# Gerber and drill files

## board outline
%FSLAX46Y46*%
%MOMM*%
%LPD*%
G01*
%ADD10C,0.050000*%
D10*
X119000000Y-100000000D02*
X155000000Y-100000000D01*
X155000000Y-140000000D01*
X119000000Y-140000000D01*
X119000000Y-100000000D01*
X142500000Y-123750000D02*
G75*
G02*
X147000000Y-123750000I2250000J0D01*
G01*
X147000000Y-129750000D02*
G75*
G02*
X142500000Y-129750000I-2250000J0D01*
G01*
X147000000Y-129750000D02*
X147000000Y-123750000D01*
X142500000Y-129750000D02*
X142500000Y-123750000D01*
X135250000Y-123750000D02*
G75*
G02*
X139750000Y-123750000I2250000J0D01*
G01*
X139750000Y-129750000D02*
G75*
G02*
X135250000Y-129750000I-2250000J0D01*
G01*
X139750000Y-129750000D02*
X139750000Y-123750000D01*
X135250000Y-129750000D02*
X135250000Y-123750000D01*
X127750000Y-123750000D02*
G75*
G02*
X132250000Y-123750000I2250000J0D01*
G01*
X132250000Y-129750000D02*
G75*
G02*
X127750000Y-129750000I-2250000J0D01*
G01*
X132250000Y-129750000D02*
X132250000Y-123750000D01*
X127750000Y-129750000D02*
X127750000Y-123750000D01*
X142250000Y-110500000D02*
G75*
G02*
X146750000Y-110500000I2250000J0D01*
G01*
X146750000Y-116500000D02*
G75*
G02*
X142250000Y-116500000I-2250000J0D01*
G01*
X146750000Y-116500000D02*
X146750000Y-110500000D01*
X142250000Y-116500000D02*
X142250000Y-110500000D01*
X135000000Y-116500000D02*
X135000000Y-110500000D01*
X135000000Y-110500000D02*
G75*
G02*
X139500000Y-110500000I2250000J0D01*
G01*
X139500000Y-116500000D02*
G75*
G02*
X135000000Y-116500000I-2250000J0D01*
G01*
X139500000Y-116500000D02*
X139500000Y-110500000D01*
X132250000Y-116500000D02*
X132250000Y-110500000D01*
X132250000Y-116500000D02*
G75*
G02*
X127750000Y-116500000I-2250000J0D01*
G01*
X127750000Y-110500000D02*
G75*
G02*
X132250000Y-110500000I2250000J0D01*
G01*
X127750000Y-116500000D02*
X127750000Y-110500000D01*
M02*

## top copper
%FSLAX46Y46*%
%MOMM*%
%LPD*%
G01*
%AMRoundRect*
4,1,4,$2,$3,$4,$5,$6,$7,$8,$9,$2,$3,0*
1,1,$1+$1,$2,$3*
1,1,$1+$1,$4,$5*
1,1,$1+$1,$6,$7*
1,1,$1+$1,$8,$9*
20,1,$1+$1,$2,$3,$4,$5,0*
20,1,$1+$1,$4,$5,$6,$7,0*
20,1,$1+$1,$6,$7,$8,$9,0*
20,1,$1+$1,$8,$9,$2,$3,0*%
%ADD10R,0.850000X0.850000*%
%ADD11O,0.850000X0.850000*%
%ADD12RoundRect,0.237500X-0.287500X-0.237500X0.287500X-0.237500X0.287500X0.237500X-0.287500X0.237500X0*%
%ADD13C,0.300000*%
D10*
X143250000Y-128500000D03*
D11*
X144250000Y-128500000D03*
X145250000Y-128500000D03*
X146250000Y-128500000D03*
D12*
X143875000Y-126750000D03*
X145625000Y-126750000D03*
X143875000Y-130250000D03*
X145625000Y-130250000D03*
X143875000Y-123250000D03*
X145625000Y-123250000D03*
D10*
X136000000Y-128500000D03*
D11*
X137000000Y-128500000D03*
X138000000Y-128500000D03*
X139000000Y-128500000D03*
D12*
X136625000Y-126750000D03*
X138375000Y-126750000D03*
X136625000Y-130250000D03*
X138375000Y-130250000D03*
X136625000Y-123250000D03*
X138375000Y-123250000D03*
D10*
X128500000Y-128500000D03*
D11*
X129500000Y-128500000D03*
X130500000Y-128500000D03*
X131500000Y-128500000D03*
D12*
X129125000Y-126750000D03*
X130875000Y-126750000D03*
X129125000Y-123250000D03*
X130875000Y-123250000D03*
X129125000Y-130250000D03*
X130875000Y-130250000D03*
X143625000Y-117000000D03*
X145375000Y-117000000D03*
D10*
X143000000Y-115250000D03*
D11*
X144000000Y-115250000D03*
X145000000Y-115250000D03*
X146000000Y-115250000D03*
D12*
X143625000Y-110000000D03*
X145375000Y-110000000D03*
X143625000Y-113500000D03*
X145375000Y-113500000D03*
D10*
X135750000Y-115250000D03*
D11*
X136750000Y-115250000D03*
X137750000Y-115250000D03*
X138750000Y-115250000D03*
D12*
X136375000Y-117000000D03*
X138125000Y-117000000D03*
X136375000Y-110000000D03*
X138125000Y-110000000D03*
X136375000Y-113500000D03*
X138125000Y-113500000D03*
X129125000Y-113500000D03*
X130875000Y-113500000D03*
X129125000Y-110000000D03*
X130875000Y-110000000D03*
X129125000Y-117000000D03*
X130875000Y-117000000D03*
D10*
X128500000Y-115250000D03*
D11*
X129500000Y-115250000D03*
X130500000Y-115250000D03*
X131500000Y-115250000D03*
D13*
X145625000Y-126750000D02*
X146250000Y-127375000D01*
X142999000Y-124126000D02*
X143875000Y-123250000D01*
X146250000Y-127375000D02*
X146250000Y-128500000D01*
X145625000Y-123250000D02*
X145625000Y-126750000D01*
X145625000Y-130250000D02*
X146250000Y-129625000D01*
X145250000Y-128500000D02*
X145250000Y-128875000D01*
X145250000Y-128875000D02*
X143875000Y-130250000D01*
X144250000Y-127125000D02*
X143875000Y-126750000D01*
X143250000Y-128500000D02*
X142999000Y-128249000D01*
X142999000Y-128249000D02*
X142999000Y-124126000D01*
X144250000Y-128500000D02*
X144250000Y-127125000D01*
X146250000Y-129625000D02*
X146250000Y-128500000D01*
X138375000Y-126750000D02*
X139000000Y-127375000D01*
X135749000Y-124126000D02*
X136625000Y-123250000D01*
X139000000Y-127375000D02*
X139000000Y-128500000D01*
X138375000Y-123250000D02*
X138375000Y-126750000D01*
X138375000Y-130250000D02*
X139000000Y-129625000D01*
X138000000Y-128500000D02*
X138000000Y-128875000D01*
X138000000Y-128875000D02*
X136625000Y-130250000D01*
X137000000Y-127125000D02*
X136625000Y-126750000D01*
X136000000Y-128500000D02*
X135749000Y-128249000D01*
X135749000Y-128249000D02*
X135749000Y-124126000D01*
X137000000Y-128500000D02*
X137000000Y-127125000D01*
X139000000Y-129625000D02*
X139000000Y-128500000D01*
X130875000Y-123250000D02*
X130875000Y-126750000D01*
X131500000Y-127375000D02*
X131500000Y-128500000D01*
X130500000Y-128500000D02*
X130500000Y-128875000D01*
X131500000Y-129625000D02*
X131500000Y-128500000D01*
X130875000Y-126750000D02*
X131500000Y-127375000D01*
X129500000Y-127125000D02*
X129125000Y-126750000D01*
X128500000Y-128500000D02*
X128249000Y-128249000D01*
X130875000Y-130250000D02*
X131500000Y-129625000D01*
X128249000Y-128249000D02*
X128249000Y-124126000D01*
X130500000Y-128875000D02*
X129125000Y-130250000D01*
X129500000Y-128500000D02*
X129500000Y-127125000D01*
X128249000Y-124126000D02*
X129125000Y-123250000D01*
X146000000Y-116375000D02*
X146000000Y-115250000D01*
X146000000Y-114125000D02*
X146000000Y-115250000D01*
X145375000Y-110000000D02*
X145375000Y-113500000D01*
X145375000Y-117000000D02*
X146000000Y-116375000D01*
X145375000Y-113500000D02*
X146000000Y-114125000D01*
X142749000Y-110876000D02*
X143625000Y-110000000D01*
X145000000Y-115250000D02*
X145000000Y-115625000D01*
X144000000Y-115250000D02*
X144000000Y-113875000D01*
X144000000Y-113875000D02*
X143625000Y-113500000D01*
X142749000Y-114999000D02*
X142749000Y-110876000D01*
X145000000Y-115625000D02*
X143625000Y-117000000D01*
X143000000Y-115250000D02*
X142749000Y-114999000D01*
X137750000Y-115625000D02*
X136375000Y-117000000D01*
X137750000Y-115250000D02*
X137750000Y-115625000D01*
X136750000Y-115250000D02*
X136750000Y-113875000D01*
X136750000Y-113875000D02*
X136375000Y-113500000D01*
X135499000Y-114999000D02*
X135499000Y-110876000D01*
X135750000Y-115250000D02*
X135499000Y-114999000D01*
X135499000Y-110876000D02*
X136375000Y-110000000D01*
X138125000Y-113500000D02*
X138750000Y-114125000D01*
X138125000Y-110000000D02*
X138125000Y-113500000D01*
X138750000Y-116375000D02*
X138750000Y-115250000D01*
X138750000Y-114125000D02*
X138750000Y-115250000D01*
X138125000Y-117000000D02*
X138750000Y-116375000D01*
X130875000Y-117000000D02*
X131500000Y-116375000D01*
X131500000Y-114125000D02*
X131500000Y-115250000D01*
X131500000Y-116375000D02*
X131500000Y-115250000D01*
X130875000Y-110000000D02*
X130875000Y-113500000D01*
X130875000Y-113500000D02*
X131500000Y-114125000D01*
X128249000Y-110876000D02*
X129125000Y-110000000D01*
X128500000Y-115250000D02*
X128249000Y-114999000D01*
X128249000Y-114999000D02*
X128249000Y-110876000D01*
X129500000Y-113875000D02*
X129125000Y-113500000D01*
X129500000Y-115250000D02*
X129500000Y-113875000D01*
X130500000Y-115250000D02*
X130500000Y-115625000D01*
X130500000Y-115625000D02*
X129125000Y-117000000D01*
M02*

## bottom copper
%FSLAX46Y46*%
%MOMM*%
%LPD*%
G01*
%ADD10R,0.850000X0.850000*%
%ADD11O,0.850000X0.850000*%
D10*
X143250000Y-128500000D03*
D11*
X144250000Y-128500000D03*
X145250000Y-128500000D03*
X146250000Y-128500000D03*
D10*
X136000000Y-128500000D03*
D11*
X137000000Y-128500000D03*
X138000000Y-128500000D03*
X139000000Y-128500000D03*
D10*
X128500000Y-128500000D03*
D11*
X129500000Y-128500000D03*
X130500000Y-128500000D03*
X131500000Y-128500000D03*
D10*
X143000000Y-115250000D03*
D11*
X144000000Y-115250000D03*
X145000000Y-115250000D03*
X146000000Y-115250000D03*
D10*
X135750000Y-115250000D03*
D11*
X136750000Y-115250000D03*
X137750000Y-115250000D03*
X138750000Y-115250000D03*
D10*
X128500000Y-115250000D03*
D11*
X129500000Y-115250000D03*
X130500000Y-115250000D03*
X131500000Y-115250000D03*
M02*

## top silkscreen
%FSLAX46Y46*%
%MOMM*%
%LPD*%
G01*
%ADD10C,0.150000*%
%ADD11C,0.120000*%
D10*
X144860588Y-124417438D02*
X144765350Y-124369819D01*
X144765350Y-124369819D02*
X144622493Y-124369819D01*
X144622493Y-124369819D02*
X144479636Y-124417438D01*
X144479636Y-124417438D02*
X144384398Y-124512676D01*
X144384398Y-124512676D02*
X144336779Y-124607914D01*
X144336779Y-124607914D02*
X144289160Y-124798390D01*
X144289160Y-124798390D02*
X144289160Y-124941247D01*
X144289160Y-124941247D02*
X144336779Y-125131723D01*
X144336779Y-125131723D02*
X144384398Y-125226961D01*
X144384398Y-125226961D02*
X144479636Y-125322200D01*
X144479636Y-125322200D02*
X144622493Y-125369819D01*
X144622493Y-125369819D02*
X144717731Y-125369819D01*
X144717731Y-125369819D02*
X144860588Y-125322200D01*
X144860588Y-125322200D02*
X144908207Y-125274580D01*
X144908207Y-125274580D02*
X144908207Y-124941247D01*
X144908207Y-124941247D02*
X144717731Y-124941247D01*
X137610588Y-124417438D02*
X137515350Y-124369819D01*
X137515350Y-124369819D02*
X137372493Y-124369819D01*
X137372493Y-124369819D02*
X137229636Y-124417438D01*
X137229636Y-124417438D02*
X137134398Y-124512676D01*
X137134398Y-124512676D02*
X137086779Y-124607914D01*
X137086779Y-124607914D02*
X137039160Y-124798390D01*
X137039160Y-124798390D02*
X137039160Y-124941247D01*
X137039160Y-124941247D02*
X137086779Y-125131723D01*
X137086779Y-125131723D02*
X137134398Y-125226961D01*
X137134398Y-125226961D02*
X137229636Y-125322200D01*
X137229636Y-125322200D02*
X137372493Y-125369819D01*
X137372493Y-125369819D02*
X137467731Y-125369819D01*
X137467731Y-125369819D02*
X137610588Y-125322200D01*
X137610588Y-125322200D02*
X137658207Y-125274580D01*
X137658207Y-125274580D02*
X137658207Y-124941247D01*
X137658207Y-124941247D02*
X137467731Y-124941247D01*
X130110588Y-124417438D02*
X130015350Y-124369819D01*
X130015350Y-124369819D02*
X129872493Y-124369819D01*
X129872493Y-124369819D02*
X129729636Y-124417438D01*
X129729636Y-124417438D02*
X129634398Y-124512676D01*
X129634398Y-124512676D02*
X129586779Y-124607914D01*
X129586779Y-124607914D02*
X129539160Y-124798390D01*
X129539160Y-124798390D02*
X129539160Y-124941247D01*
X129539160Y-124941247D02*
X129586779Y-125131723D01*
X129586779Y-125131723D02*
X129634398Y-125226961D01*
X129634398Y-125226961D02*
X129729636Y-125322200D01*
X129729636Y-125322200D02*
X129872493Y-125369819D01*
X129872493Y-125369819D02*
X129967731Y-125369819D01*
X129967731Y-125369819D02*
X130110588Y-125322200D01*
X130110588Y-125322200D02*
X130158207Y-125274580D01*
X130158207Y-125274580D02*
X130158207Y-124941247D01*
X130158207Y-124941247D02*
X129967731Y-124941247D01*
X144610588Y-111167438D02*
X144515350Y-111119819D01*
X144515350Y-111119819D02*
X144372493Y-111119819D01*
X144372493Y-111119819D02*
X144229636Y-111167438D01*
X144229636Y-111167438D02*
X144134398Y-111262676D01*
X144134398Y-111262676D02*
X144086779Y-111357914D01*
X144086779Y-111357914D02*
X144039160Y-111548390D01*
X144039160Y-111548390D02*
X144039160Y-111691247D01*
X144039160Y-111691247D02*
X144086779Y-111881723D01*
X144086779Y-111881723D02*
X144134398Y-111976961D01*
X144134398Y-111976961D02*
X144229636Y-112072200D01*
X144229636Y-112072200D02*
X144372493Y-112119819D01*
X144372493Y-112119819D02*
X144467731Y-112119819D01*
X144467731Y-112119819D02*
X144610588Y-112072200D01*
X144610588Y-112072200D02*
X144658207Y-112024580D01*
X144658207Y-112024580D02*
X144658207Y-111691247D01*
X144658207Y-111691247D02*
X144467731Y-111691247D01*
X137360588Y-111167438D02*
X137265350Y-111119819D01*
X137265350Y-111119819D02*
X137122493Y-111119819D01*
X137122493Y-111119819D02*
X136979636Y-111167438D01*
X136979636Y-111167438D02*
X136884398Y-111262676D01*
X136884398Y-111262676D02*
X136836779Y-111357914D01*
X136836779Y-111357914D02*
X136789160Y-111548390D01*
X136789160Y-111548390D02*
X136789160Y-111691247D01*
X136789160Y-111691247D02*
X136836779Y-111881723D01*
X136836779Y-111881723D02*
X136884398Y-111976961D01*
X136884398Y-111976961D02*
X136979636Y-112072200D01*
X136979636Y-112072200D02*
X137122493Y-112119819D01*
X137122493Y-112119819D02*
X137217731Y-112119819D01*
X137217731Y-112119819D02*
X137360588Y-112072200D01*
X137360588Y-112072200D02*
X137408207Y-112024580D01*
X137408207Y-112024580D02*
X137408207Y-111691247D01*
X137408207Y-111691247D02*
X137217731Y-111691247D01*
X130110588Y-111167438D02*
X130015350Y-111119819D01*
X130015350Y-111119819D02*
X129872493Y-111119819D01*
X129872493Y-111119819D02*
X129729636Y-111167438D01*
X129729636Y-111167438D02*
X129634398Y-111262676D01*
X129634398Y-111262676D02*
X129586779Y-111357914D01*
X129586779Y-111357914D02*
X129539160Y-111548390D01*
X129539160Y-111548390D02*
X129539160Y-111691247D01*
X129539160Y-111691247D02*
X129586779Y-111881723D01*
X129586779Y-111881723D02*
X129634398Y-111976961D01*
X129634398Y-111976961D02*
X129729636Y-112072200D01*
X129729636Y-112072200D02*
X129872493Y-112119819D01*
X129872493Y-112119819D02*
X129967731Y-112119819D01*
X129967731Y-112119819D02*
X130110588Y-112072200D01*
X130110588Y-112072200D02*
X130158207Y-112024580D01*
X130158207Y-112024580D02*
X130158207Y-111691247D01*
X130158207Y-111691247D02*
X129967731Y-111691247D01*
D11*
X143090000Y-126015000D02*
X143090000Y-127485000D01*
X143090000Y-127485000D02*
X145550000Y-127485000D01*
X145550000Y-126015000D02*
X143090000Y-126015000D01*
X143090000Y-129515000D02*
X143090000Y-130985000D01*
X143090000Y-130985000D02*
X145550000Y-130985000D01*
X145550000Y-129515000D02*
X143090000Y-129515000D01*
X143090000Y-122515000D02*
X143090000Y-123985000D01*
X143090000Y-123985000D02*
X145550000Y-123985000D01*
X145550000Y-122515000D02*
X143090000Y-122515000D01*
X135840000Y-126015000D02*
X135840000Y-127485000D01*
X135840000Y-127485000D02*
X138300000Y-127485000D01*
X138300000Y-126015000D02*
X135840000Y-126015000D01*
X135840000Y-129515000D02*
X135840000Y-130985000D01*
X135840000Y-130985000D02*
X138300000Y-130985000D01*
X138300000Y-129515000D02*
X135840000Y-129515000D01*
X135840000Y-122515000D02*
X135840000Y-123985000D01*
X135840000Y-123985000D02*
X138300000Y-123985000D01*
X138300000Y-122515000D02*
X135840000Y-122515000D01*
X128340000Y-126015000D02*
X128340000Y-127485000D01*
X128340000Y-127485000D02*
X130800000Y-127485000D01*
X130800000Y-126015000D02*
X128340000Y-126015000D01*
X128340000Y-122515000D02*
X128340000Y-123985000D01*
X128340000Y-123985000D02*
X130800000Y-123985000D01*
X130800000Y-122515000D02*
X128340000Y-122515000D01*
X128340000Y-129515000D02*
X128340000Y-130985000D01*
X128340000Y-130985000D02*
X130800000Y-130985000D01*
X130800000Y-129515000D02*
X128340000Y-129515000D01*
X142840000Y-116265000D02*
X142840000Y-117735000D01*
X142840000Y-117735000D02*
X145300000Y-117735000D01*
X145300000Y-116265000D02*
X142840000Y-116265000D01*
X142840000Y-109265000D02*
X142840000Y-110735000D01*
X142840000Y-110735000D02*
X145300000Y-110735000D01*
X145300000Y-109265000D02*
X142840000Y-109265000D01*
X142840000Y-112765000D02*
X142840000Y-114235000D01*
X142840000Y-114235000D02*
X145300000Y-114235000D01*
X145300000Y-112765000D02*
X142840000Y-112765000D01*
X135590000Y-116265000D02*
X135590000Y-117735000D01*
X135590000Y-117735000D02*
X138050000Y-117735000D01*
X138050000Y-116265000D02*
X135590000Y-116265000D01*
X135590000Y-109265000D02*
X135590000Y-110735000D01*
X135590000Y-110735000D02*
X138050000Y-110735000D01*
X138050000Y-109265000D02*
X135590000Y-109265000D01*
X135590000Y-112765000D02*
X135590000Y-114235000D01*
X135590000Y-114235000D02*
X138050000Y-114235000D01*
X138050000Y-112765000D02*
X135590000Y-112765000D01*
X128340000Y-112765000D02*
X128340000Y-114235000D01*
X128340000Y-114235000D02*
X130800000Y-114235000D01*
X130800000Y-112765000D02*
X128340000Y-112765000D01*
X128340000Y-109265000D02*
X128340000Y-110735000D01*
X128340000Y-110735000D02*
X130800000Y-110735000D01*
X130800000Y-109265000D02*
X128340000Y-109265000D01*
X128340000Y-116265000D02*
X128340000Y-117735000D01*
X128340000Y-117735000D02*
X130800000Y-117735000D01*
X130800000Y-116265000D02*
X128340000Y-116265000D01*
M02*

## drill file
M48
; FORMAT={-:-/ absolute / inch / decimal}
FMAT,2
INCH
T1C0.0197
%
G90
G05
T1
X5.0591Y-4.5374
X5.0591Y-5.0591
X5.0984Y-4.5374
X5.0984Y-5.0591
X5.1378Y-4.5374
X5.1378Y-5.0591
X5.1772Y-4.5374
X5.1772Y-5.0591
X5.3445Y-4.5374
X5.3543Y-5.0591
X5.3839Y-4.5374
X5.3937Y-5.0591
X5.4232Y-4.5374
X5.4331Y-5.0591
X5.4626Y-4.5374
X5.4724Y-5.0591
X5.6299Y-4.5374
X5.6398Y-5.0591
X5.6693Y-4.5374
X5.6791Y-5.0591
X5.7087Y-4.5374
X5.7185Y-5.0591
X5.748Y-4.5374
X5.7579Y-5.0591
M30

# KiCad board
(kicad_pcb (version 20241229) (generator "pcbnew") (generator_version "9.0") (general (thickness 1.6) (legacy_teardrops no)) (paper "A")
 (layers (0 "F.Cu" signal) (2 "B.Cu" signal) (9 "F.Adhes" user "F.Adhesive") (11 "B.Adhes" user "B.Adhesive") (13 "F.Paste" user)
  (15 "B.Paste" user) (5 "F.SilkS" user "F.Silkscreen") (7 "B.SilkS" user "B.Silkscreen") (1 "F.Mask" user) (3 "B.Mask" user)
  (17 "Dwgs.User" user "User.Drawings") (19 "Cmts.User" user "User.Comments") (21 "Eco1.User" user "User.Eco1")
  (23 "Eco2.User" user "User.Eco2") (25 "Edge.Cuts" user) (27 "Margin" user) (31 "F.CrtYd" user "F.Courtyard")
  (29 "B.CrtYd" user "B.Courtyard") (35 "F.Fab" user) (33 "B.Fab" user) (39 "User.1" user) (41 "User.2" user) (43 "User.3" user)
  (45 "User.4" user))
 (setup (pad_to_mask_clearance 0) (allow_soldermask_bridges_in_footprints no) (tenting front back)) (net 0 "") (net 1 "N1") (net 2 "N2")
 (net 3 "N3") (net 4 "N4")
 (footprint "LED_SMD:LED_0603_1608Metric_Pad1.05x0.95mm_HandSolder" (layer "F.Cu") (at 144.5 113.5)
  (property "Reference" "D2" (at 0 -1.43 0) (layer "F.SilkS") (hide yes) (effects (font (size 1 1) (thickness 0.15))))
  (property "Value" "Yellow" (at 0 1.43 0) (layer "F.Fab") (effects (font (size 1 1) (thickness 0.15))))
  (fp_line (start -1.66 -0.735) (end -1.66 0.735) (stroke (width 0.12) (type solid)) (layer "F.SilkS"))
  (fp_line (start -1.66 0.735) (end 0.8 0.735) (stroke (width 0.12) (type solid)) (layer "F.SilkS"))
  (fp_line (start 0.8 -0.735) (end -1.66 -0.735) (stroke (width 0.12) (type solid)) (layer "F.SilkS"))
  (pad "1" smd roundrect (at -0.875 0) (size 1.05 0.95) (layers "F.Cu" "F.Mask" "F.Paste") (roundrect_rratio 0.25) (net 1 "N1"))
  (pad "2" smd roundrect (at 0.875 0) (size 1.05 0.95) (layers "F.Cu" "F.Mask" "F.Paste") (roundrect_rratio 0.25) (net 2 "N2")))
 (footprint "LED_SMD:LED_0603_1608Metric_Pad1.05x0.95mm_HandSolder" (layer "F.Cu") (at 137.25 113.5)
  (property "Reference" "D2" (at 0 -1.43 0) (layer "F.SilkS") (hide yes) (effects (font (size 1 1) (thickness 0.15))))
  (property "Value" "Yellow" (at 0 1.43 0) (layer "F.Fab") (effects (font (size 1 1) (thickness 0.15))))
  (fp_line (start -1.66 -0.735) (end -1.66 0.735) (stroke (width 0.12) (type solid)) (layer "F.SilkS"))
  (fp_line (start -1.66 0.735) (end 0.8 0.735) (stroke (width 0.12) (type solid)) (layer "F.SilkS"))
  (fp_line (start 0.8 -0.735) (end -1.66 -0.735) (stroke (width 0.12) (type solid)) (layer "F.SilkS"))
  (pad "1" smd roundrect (at -0.875 0) (size 1.05 0.95) (layers "F.Cu" "F.Mask" "F.Paste") (roundrect_rratio 0.25) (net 1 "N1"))
  (pad "2" smd roundrect (at 0.875 0) (size 1.05 0.95) (layers "F.Cu" "F.Mask" "F.Paste") (roundrect_rratio 0.25) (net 2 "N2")))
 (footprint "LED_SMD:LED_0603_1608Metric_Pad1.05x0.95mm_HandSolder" (layer "F.Cu") (at 137.5 126.75)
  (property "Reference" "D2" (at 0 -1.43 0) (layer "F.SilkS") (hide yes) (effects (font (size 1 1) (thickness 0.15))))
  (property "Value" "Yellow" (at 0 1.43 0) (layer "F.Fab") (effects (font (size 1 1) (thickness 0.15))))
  (fp_line (start -1.66 -0.735) (end -1.66 0.735) (stroke (width 0.12) (type solid)) (layer "F.SilkS"))
  (fp_line (start -1.66 0.735) (end 0.8 0.735) (stroke (width 0.12) (type solid)) (layer "F.SilkS"))
  (fp_line (start 0.8 -0.735) (end -1.66 -0.735) (stroke (width 0.12) (type solid)) (layer "F.SilkS"))
  (pad "1" smd roundrect (at -0.875 0) (size 1.05 0.95) (layers "F.Cu" "F.Mask" "F.Paste") (roundrect_rratio 0.25) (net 1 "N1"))
  (pad "2" smd roundrect (at 0.875 0) (size 1.05 0.95) (layers "F.Cu" "F.Mask" "F.Paste") (roundrect_rratio 0.25) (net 2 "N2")))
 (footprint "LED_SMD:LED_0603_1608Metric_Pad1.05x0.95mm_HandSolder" (layer "F.Cu") (at 130 123.25)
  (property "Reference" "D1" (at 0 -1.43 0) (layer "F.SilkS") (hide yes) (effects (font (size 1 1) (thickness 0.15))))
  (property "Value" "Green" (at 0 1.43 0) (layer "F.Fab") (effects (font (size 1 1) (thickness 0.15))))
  (fp_line (start -1.66 -0.735) (end -1.66 0.735) (stroke (width 0.12) (type solid)) (layer "F.SilkS"))
  (fp_line (start -1.66 0.735) (end 0.8 0.735) (stroke (width 0.12) (type solid)) (layer "F.SilkS"))
  (fp_line (start 0.8 -0.735) (end -1.66 -0.735) (stroke (width 0.12) (type solid)) (layer "F.SilkS"))
  (pad "1" smd roundrect (at -0.875 0) (size 1.05 0.95) (layers "F.Cu" "F.Mask" "F.Paste") (roundrect_rratio 0.25) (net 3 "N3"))
  (pad "2" smd roundrect (at 0.875 0) (size 1.05 0.95) (layers "F.Cu" "F.Mask" "F.Paste") (roundrect_rratio 0.25) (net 2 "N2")))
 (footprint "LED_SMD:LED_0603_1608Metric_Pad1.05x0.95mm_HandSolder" (layer "F.Cu") (at 130 130.25)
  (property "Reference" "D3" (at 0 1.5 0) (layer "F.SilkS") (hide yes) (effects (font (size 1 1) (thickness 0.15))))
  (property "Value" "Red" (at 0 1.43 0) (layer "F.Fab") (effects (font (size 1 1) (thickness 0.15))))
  (fp_line (start -1.66 -0.735) (end -1.66 0.735) (stroke (width 0.12) (type solid)) (layer "F.SilkS"))
  (fp_line (start -1.66 0.735) (end 0.8 0.735) (stroke (width 0.12) (type solid)) (layer "F.SilkS"))
  (fp_line (start 0.8 -0.735) (end -1.66 -0.735) (stroke (width 0.12) (type solid)) (layer "F.SilkS"))
  (pad "1" smd roundrect (at -0.875 0) (size 1.05 0.95) (layers "F.Cu" "F.Mask" "F.Paste") (roundrect_rratio 0.25) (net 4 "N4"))
  (pad "2" smd roundrect (at 0.875 0) (size 1.05 0.95) (layers "F.Cu" "F.Mask" "F.Paste") (roundrect_rratio 0.25) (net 2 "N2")))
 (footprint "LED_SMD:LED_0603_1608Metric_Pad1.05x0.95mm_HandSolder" (layer "F.Cu") (at 144.5 110)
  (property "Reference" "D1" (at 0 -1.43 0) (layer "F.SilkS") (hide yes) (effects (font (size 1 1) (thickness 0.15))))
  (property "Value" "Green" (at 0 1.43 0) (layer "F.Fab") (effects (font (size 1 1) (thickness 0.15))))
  (fp_line (start -1.66 -0.735) (end -1.66 0.735) (stroke (width 0.12) (type solid)) (layer "F.SilkS"))
  (fp_line (start -1.66 0.735) (end 0.8 0.735) (stroke (width 0.12) (type solid)) (layer "F.SilkS"))
  (fp_line (start 0.8 -0.735) (end -1.66 -0.735) (stroke (width 0.12) (type solid)) (layer "F.SilkS"))
  (pad "1" smd roundrect (at -0.875 0) (size 1.05 0.95) (layers "F.Cu" "F.Mask" "F.Paste") (roundrect_rratio 0.25) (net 3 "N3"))
  (pad "2" smd roundrect (at 0.875 0) (size 1.05 0.95) (layers "F.Cu" "F.Mask" "F.Paste") (roundrect_rratio 0.25) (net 2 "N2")))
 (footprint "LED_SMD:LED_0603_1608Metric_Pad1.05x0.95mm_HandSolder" (layer "F.Cu") (at 137.5 123.25)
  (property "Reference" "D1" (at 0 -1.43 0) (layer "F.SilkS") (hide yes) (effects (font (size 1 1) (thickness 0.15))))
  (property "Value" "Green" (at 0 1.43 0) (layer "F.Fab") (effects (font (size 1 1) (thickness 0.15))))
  (fp_line (start -1.66 -0.735) (end -1.66 0.735) (stroke (width 0.12) (type solid)) (layer "F.SilkS"))
  (fp_line (start -1.66 0.735) (end 0.8 0.735) (stroke (width 0.12) (type solid)) (layer "F.SilkS"))
  (fp_line (start 0.8 -0.735) (end -1.66 -0.735) (stroke (width 0.12) (type solid)) (layer "F.SilkS"))
  (pad "1" smd roundrect (at -0.875 0) (size 1.05 0.95) (layers "F.Cu" "F.Mask" "F.Paste") (roundrect_rratio 0.25) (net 3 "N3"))
  (pad "2" smd roundrect (at 0.875 0) (size 1.05 0.95) (layers "F.Cu" "F.Mask" "F.Paste") (roundrect_rratio 0.25) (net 2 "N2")))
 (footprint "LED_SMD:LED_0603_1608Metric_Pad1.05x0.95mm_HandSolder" (layer "F.Cu") (at 144.75 123.25)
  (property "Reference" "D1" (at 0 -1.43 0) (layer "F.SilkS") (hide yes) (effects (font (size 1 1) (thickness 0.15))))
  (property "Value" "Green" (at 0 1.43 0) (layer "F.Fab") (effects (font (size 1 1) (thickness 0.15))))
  (fp_line (start -1.66 -0.735) (end -1.66 0.735) (stroke (width 0.12) (type solid)) (layer "F.SilkS"))
  (fp_line (start -1.66 0.735) (end 0.8 0.735) (stroke (width 0.12) (type solid)) (layer "F.SilkS"))
  (fp_line (start 0.8 -0.735) (end -1.66 -0.735) (stroke (width 0.12) (type solid)) (layer "F.SilkS"))
  (pad "1" smd roundrect (at -0.875 0) (size 1.05 0.95) (layers "F.Cu" "F.Mask" "F.Paste") (roundrect_rratio 0.25) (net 3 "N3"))
  (pad "2" smd roundrect (at 0.875 0) (size 1.05 0.95) (layers "F.Cu" "F.Mask" "F.Paste") (roundrect_rratio 0.25) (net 2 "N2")))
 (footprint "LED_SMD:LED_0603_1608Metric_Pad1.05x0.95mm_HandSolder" (layer "F.Cu") (at 144.5 117)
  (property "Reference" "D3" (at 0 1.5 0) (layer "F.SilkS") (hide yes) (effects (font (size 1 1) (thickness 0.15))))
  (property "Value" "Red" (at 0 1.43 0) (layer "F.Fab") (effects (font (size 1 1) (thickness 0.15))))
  (fp_line (start -1.66 -0.735) (end -1.66 0.735) (stroke (width 0.12) (type solid)) (layer "F.SilkS"))
  (fp_line (start -1.66 0.735) (end 0.8 0.735) (stroke (width 0.12) (type solid)) (layer "F.SilkS"))
  (fp_line (start 0.8 -0.735) (end -1.66 -0.735) (stroke (width 0.12) (type solid)) (layer "F.SilkS"))
  (pad "1" smd roundrect (at -0.875 0) (size 1.05 0.95) (layers "F.Cu" "F.Mask" "F.Paste") (roundrect_rratio 0.25) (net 4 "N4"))
  (pad "2" smd roundrect (at 0.875 0) (size 1.05 0.95) (layers "F.Cu" "F.Mask" "F.Paste") (roundrect_rratio 0.25) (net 2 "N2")))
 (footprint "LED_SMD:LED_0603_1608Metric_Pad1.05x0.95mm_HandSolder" (layer "F.Cu") (at 137.25 110)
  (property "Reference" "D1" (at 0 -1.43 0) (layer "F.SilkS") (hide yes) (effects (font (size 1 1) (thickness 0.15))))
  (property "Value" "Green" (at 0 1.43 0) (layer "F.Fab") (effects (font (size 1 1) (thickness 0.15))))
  (fp_line (start -1.66 -0.735) (end -1.66 0.735) (stroke (width 0.12) (type solid)) (layer "F.SilkS"))
  (fp_line (start -1.66 0.735) (end 0.8 0.735) (stroke (width 0.12) (type solid)) (layer "F.SilkS"))
  (fp_line (start 0.8 -0.735) (end -1.66 -0.735) (stroke (width 0.12) (type solid)) (layer "F.SilkS"))
  (pad "1" smd roundrect (at -0.875 0) (size 1.05 0.95) (layers "F.Cu" "F.Mask" "F.Paste") (roundrect_rratio 0.25) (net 3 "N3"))
  (pad "2" smd roundrect (at 0.875 0) (size 1.05 0.95) (layers "F.Cu" "F.Mask" "F.Paste") (roundrect_rratio 0.25) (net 2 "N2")))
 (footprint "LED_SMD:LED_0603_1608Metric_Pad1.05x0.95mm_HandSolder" (layer "F.Cu") (at 130 113.5)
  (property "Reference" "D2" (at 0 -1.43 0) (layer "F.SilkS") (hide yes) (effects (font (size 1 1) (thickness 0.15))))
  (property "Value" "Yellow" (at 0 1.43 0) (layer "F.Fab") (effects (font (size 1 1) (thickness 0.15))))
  (fp_line (start -1.66 -0.735) (end -1.66 0.735) (stroke (width 0.12) (type solid)) (layer "F.SilkS"))
  (fp_line (start -1.66 0.735) (end 0.8 0.735) (stroke (width 0.12) (type solid)) (layer "F.SilkS"))
  (fp_line (start 0.8 -0.735) (end -1.66 -0.735) (stroke (width 0.12) (type solid)) (layer "F.SilkS"))
  (pad "1" smd roundrect (at -0.875 0) (size 1.05 0.95) (layers "F.Cu" "F.Mask" "F.Paste") (roundrect_rratio 0.25) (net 1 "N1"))
  (pad "2" smd roundrect (at 0.875 0) (size 1.05 0.95) (layers "F.Cu" "F.Mask" "F.Paste") (roundrect_rratio 0.25) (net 2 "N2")))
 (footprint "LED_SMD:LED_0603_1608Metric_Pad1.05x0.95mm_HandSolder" (layer "F.Cu") (at 130 126.75)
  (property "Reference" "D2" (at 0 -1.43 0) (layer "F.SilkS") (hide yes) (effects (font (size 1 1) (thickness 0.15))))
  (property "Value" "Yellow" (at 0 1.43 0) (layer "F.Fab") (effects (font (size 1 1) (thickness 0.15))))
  (fp_line (start -1.66 -0.735) (end -1.66 0.735) (stroke (width 0.12) (type solid)) (layer "F.SilkS"))
  (fp_line (start -1.66 0.735) (end 0.8 0.735) (stroke (width 0.12) (type solid)) (layer "F.SilkS"))
  (fp_line (start 0.8 -0.735) (end -1.66 -0.735) (stroke (width 0.12) (type solid)) (layer "F.SilkS"))
  (pad "1" smd roundrect (at -0.875 0) (size 1.05 0.95) (layers "F.Cu" "F.Mask" "F.Paste") (roundrect_rratio 0.25) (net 1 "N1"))
  (pad "2" smd roundrect (at 0.875 0) (size 1.05 0.95) (layers "F.Cu" "F.Mask" "F.Paste") (roundrect_rratio 0.25) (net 2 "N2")))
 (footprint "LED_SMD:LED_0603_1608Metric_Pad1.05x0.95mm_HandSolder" (layer "F.Cu") (at 144.75 126.75)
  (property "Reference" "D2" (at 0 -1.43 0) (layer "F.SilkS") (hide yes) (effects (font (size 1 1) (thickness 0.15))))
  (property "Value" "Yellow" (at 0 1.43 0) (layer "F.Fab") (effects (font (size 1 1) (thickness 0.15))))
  (fp_line (start -1.66 -0.735) (end -1.66 0.735) (stroke (width 0.12) (type solid)) (layer "F.SilkS"))
  (fp_line (start -1.66 0.735) (end 0.8 0.735) (stroke (width 0.12) (type solid)) (layer "F.SilkS"))
  (fp_line (start 0.8 -0.735) (end -1.66 -0.735) (stroke (width 0.12) (type solid)) (layer "F.SilkS"))
  (pad "1" smd roundrect (at -0.875 0) (size 1.05 0.95) (layers "F.Cu" "F.Mask" "F.Paste") (roundrect_rratio 0.25) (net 1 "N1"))
  (pad "2" smd roundrect (at 0.875 0) (size 1.05 0.95) (layers "F.Cu" "F.Mask" "F.Paste") (roundrect_rratio 0.25) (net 2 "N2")))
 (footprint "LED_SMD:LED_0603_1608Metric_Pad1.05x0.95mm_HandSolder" (layer "F.Cu") (at 137.5 130.25)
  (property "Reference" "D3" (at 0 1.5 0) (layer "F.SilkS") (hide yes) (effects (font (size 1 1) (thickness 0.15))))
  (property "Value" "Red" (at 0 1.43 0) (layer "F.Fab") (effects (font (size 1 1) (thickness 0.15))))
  (fp_line (start -1.66 -0.735) (end -1.66 0.735) (stroke (width 0.12) (type solid)) (layer "F.SilkS"))
  (fp_line (start -1.66 0.735) (end 0.8 0.735) (stroke (width 0.12) (type solid)) (layer "F.SilkS"))
  (fp_line (start 0.8 -0.735) (end -1.66 -0.735) (stroke (width 0.12) (type solid)) (layer "F.SilkS"))
  (pad "1" smd roundrect (at -0.875 0) (size 1.05 0.95) (layers "F.Cu" "F.Mask" "F.Paste") (roundrect_rratio 0.25) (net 4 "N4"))
  (pad "2" smd roundrect (at 0.875 0) (size 1.05 0.95) (layers "F.Cu" "F.Mask" "F.Paste") (roundrect_rratio 0.25) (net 2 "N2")))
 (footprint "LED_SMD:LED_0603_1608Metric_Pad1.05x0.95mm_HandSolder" (layer "F.Cu") (at 137.25 117)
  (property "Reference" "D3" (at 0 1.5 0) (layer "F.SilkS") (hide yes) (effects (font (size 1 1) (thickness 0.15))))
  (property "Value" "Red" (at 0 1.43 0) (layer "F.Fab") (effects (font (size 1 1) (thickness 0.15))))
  (fp_line (start -1.66 -0.735) (end -1.66 0.735) (stroke (width 0.12) (type solid)) (layer "F.SilkS"))
  (fp_line (start -1.66 0.735) (end 0.8 0.735) (stroke (width 0.12) (type solid)) (layer "F.SilkS"))
  (fp_line (start 0.8 -0.735) (end -1.66 -0.735) (stroke (width 0.12) (type solid)) (layer "F.SilkS"))
  (pad "1" smd roundrect (at -0.875 0) (size 1.05 0.95) (layers "F.Cu" "F.Mask" "F.Paste") (roundrect_rratio 0.25) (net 4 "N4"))
  (pad "2" smd roundrect (at 0.875 0) (size 1.05 0.95) (layers "F.Cu" "F.Mask" "F.Paste") (roundrect_rratio 0.25) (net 2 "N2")))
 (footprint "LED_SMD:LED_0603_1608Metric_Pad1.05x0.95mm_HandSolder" (layer "F.Cu") (at 130 110)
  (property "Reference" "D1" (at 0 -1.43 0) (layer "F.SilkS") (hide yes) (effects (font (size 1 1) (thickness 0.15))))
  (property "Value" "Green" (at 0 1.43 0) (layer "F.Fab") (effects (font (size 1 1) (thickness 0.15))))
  (fp_line (start -1.66 -0.735) (end -1.66 0.735) (stroke (width 0.12) (type solid)) (layer "F.SilkS"))
  (fp_line (start -1.66 0.735) (end 0.8 0.735) (stroke (width 0.12) (type solid)) (layer "F.SilkS"))
  (fp_line (start 0.8 -0.735) (end -1.66 -0.735) (stroke (width 0.12) (type solid)) (layer "F.SilkS"))
  (pad "1" smd roundrect (at -0.875 0) (size 1.05 0.95) (layers "F.Cu" "F.Mask" "F.Paste") (roundrect_rratio 0.25) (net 3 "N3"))
  (pad "2" smd roundrect (at 0.875 0) (size 1.05 0.95) (layers "F.Cu" "F.Mask" "F.Paste") (roundrect_rratio 0.25) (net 2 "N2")))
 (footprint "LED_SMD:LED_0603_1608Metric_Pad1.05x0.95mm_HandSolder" (layer "F.Cu") (at 130 117)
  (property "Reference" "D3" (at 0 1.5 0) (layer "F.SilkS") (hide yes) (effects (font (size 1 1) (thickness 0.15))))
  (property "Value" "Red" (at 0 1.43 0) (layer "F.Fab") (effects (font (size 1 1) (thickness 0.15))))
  (fp_line (start -1.66 -0.735) (end -1.66 0.735) (stroke (width 0.12) (type solid)) (layer "F.SilkS"))
  (fp_line (start -1.66 0.735) (end 0.8 0.735) (stroke (width 0.12) (type solid)) (layer "F.SilkS"))
  (fp_line (start 0.8 -0.735) (end -1.66 -0.735) (stroke (width 0.12) (type solid)) (layer "F.SilkS"))
  (pad "1" smd roundrect (at -0.875 0) (size 1.05 0.95) (layers "F.Cu" "F.Mask" "F.Paste") (roundrect_rratio 0.25) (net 4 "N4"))
  (pad "2" smd roundrect (at 0.875 0) (size 1.05 0.95) (layers "F.Cu" "F.Mask" "F.Paste") (roundrect_rratio 0.25) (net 2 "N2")))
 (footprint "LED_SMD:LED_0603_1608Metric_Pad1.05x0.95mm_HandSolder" (layer "F.Cu") (at 144.75 130.25)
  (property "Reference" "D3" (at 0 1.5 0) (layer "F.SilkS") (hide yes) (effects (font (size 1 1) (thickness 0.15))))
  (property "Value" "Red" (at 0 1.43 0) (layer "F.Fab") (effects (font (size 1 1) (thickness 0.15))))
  (fp_line (start -1.66 -0.735) (end -1.66 0.735) (stroke (width 0.12) (type solid)) (layer "F.SilkS"))
  (fp_line (start -1.66 0.735) (end 0.8 0.735) (stroke (width 0.12) (type solid)) (layer "F.SilkS"))
  (fp_line (start 0.8 -0.735) (end -1.66 -0.735) (stroke (width 0.12) (type solid)) (layer "F.SilkS"))
  (pad "1" smd roundrect (at -0.875 0) (size 1.05 0.95) (layers "F.Cu" "F.Mask" "F.Paste") (roundrect_rratio 0.25) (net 4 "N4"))
  (pad "2" smd roundrect (at 0.875 0) (size 1.05 0.95) (layers "F.Cu" "F.Mask" "F.Paste") (roundrect_rratio 0.25) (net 2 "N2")))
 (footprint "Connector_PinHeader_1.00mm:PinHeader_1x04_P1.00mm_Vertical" (layer "B.Cu") (at 128.5 128.5 -90)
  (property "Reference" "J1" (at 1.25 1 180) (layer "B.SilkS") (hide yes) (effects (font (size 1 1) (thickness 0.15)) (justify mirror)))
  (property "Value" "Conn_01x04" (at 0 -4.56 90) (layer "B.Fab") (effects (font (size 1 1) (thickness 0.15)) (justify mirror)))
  (pad "1" thru_hole rect (at 0 0 270) (size 0.85 0.85) (drill 0.5) (layers "*.Cu" "*.Mask") (remove_unused_layers no) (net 3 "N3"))
  (pad "2" thru_hole oval (at 0 -1 270) (size 0.85 0.85) (drill 0.5) (layers "*.Cu" "*.Mask") (remove_unused_layers no) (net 1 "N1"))
  (pad "3" thru_hole oval (at 0 -2 270) (size 0.85 0.85) (drill 0.5) (layers "*.Cu" "*.Mask") (remove_unused_layers no) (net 4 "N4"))
  (pad "4" thru_hole oval (at 0 -3 270) (size 0.85 0.85) (drill 0.5) (layers "*.Cu" "*.Mask") (remove_unused_layers no) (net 2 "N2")))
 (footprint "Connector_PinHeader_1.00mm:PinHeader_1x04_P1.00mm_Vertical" (layer "B.Cu") (at 143.25 128.5 -90)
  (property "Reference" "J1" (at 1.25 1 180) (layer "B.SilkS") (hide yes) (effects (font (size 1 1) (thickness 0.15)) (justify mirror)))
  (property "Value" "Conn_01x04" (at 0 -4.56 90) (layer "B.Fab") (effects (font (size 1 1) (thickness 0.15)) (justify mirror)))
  (pad "1" thru_hole rect (at 0 0 270) (size 0.85 0.85) (drill 0.5) (layers "*.Cu" "*.Mask") (remove_unused_layers no) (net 3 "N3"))
  (pad "2" thru_hole oval (at 0 -1 270) (size 0.85 0.85) (drill 0.5) (layers "*.Cu" "*.Mask") (remove_unused_layers no) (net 1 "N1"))
  (pad "3" thru_hole oval (at 0 -2 270) (size 0.85 0.85) (drill 0.5) (layers "*.Cu" "*.Mask") (remove_unused_layers no) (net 4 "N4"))
  (pad "4" thru_hole oval (at 0 -3 270) (size 0.85 0.85) (drill 0.5) (layers "*.Cu" "*.Mask") (remove_unused_layers no) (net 2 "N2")))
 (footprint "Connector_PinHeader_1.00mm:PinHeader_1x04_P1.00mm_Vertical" (layer "B.Cu") (at 136 128.5 -90)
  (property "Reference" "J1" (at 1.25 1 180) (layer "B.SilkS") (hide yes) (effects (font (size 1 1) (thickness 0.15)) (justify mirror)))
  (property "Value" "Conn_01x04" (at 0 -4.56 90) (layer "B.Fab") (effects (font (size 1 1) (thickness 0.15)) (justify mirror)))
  (pad "1" thru_hole rect (at 0 0 270) (size 0.85 0.85) (drill 0.5) (layers "*.Cu" "*.Mask") (remove_unused_layers no) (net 3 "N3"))
  (pad "2" thru_hole oval (at 0 -1 270) (size 0.85 0.85) (drill 0.5) (layers "*.Cu" "*.Mask") (remove_unused_layers no) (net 1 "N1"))
  (pad "3" thru_hole oval (at 0 -2 270) (size 0.85 0.85) (drill 0.5) (layers "*.Cu" "*.Mask") (remove_unused_layers no) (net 4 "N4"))
  (pad "4" thru_hole oval (at 0 -3 270) (size 0.85 0.85) (drill 0.5) (layers "*.Cu" "*.Mask") (remove_unused_layers no) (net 2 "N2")))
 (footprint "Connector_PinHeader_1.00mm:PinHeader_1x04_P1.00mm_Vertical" (layer "B.Cu") (at 128.5 115.25 -90)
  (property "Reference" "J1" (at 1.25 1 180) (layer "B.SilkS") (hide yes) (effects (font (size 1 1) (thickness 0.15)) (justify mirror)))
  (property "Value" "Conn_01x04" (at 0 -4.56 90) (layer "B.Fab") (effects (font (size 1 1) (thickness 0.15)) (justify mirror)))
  (pad "1" thru_hole rect (at 0 0 270) (size 0.85 0.85) (drill 0.5) (layers "*.Cu" "*.Mask") (remove_unused_layers no) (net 3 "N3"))
  (pad "2" thru_hole oval (at 0 -1 270) (size 0.85 0.85) (drill 0.5) (layers "*.Cu" "*.Mask") (remove_unused_layers no) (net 1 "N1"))
  (pad "3" thru_hole oval (at 0 -2 270) (size 0.85 0.85) (drill 0.5) (layers "*.Cu" "*.Mask") (remove_unused_layers no) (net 4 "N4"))
  (pad "4" thru_hole oval (at 0 -3 270) (size 0.85 0.85) (drill 0.5) (layers "*.Cu" "*.Mask") (remove_unused_layers no) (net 2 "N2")))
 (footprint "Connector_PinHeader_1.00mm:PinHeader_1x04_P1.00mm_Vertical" (layer "B.Cu") (at 135.75 115.25 -90)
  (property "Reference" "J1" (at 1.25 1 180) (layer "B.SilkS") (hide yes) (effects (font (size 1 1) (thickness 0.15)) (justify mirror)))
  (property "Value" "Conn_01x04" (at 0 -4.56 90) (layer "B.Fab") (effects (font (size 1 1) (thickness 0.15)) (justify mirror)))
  (pad "1" thru_hole rect (at 0 0 270) (size 0.85 0.85) (drill 0.5) (layers "*.Cu" "*.Mask") (remove_unused_layers no) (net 3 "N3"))
  (pad "2" thru_hole oval (at 0 -1 270) (size 0.85 0.85) (drill 0.5) (layers "*.Cu" "*.Mask") (remove_unused_layers no) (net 1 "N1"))
  (pad "3" thru_hole oval (at 0 -2 270) (size 0.85 0.85) (drill 0.5) (layers "*.Cu" "*.Mask") (remove_unused_layers no) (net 4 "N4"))
  (pad "4" thru_hole oval (at 0 -3 270) (size 0.85 0.85) (drill 0.5) (layers "*.Cu" "*.Mask") (remove_unused_layers no) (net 2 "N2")))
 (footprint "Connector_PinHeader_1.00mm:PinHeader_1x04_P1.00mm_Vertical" (layer "B.Cu") (at 143 115.25 -90)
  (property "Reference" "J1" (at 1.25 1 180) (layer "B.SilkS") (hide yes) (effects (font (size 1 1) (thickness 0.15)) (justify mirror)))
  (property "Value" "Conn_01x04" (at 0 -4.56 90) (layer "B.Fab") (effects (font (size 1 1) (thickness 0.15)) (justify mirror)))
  (pad "1" thru_hole rect (at 0 0 270) (size 0.85 0.85) (drill 0.5) (layers "*.Cu" "*.Mask") (remove_unused_layers no) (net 3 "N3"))
  (pad "2" thru_hole oval (at 0 -1 270) (size 0.85 0.85) (drill 0.5) (layers "*.Cu" "*.Mask") (remove_unused_layers no) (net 1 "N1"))
  (pad "3" thru_hole oval (at 0 -2 270) (size 0.85 0.85) (drill 0.5) (layers "*.Cu" "*.Mask") (remove_unused_layers no) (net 4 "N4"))
  (pad "4" thru_hole oval (at 0 -3 270) (size 0.85 0.85) (drill 0.5) (layers "*.Cu" "*.Mask") (remove_unused_layers no) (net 2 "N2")))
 (gr_arc (start 139.5 116.5) (mid 137.25 118.75) (end 135 116.5) (stroke (width 0.05) (type default)) (layer "Edge.Cuts"))
 (gr_line (start 142.25 116.5) (end 142.25 110.5) (stroke (width 0.05) (type default)) (layer "Edge.Cuts"))
 (gr_line (start 135 116.5) (end 135 110.5) (stroke (width 0.05) (type default)) (layer "Edge.Cuts"))
 (gr_arc (start 147 129.75) (mid 144.75 132) (end 142.5 129.75) (stroke (width 0.05) (type default)) (layer "Edge.Cuts"))
 (gr_line (start 132.25 116.5) (end 132.25 110.5) (stroke (width 0.05) (type default)) (layer "Edge.Cuts"))
 (gr_line (start 146.75 116.5) (end 146.75 110.5) (stroke (width 0.05) (type default)) (layer "Edge.Cuts"))
 (gr_arc (start 142.5 123.75) (mid 144.75 121.5) (end 147 123.75) (stroke (width 0.05) (type default)) (layer "Edge.Cuts"))
 (gr_line (start 142.5 129.75) (end 142.5 123.75) (stroke (width 0.05) (type default)) (layer "Edge.Cuts"))
 (gr_arc (start 132.25 129.75) (mid 130 132) (end 127.75 129.75) (stroke (width 0.05) (type default)) (layer "Edge.Cuts"))
 (gr_arc (start 127.75 123.75) (mid 130 121.5) (end 132.25 123.75) (stroke (width 0.05) (type default)) (layer "Edge.Cuts"))
 (gr_rect (start 119 100) (end 155 140) (stroke (width 0.05) (type default)) (fill no) (layer "Edge.Cuts"))
 (gr_line (start 135.25 129.75) (end 135.25 123.75) (stroke (width 0.05) (type default)) (layer "Edge.Cuts"))
 (gr_arc (start 139.75 129.75) (mid 137.5 132) (end 135.25 129.75) (stroke (width 0.05) (type default)) (layer "Edge.Cuts"))
 (gr_arc (start 132.25 116.5) (mid 130 118.75) (end 127.75 116.5) (stroke (width 0.05) (type default)) (layer "Edge.Cuts"))
 (gr_arc (start 146.75 116.5) (mid 144.5 118.75) (end 142.25 116.5) (stroke (width 0.05) (type default)) (layer "Edge.Cuts"))
 (gr_arc (start 135.25 123.75) (mid 137.5 121.5) (end 139.75 123.75) (stroke (width 0.05) (type default)) (layer "Edge.Cuts"))
 (gr_arc (start 127.75 110.5) (mid 130 108.25) (end 132.25 110.5) (stroke (width 0.05) (type default)) (layer "Edge.Cuts"))
 (gr_line (start 139.5 116.5) (end 139.5 110.5) (stroke (width 0.05) (type default)) (layer "Edge.Cuts"))
 (gr_line (start 147 129.75) (end 147 123.75) (stroke (width 0.05) (type default)) (layer "Edge.Cuts"))
 (gr_line (start 127.75 116.5) (end 127.75 110.5) (stroke (width 0.05) (type default)) (layer "Edge.Cuts"))
 (gr_line (start 139.75 129.75) (end 139.75 123.75) (stroke (width 0.05) (type default)) (layer "Edge.Cuts"))
 (gr_arc (start 135 110.5) (mid 137.25 108.25) (end 139.5 110.5) (stroke (width 0.05) (type default)) (layer "Edge.Cuts"))
 (gr_arc (start 142.25 110.5) (mid 144.5 108.25) (end 146.75 110.5) (stroke (width 0.05) (type default)) (layer "Edge.Cuts"))
 (gr_line (start 132.25 129.75) (end 132.25 123.75) (stroke (width 0.05) (type default)) (layer "Edge.Cuts"))
 (gr_line (start 127.75 129.75) (end 127.75 123.75) (stroke (width 0.05) (type default)) (layer "Edge.Cuts"))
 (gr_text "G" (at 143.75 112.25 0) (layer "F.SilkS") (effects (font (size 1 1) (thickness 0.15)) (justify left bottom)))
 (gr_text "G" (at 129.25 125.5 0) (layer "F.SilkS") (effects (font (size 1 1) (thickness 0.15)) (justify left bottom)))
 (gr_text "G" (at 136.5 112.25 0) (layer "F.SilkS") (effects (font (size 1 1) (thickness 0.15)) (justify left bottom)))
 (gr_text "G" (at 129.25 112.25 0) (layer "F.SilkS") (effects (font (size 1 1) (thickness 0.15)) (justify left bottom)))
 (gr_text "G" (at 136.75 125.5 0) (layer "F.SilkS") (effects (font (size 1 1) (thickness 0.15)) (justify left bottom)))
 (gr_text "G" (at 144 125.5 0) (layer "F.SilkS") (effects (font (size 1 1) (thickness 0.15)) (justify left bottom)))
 (segment (start 138.375 123.25) (end 138.375 126.75) (width 0.3) (layer "F.Cu") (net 2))
 (segment (start 130.875 117) (end 131.5 116.375) (width 0.3) (layer "F.Cu") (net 2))
 (segment (start 138.375 130.25) (end 139 129.625) (width 0.3) (layer "F.Cu") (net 2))
 (segment (start 138.75 116.375) (end 138.75 115.25) (width 0.3) (layer "F.Cu") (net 2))
 (segment (start 131.5 114.125) (end 131.5 115.25) (width 0.3) (layer "F.Cu") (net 2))
 (segment (start 145.375 117) (end 146 116.375) (width 0.3) (layer "F.Cu") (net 2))
 (segment (start 138.125 110) (end 138.125 113.5) (width 0.3) (layer "F.Cu") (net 2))
 (segment (start 130.875 126.75) (end 131.5 127.375) (width 0.3) (layer "F.Cu") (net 2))
 (segment (start 131.5 116.375) (end 131.5 115.25) (width 0.3) (layer "F.Cu") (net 2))
 (segment (start 139 129.625) (end 139 128.5) (width 0.3) (layer "F.Cu") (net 2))
 (segment (start 130.875 110) (end 130.875 113.5) (width 0.3) (layer "F.Cu") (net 2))
 (segment (start 131.5 129.625) (end 131.5 128.5) (width 0.3) (layer "F.Cu") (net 2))
 (segment (start 139 127.375) (end 139 128.5) (width 0.3) (layer "F.Cu") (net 2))
 (segment (start 138.125 113.5) (end 138.75 114.125) (width 0.3) (layer "F.Cu") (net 2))
 (segment (start 145.625 123.25) (end 145.625 126.75) (width 0.3) (layer "F.Cu") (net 2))
 (segment (start 145.375 110) (end 145.375 113.5) (width 0.3) (layer "F.Cu") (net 2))
 (segment (start 145.625 130.25) (end 146.25 129.625) (width 0.3) (layer "F.Cu") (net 2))
 (segment (start 138.75 114.125) (end 138.75 115.25) (width 0.3) (layer "F.Cu") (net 2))
 (segment (start 146 114.125) (end 146 115.25) (width 0.3) (layer "F.Cu") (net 2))
 (segment (start 130.875 123.25) (end 130.875 126.75) (width 0.3) (layer "F.Cu") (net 2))
 (segment (start 145.375 113.5) (end 146 114.125) (width 0.3) (layer "F.Cu") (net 2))
 (segment (start 145.625 126.75) (end 146.25 127.375) (width 0.3) (layer "F.Cu") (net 2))
 (segment (start 146 116.375) (end 146 115.25) (width 0.3) (layer "F.Cu") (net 2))
 (segment (start 138.375 126.75) (end 139 127.375) (width 0.3) (layer "F.Cu") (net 2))
 (segment (start 130.875 113.5) (end 131.5 114.125) (width 0.3) (layer "F.Cu") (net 2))
 (segment (start 131.5 127.375) (end 131.5 128.5) (width 0.3) (layer "F.Cu") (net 2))
 (segment (start 138.125 117) (end 138.75 116.375) (width 0.3) (layer "F.Cu") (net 2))
 (segment (start 146.25 127.375) (end 146.25 128.5) (width 0.3) (layer "F.Cu") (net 2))
 (segment (start 130.875 130.25) (end 131.5 129.625) (width 0.3) (layer "F.Cu") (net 2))
 (segment (start 146.25 129.625) (end 146.25 128.5) (width 0.3) (layer "F.Cu") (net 2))
 (segment (start 135.499 110.876) (end 136.375 110) (width 0.3) (layer "F.Cu") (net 3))
 (segment (start 142.749 110.876) (end 143.625 110) (width 0.3) (layer "F.Cu") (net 3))
 (segment (start 135.749 128.249) (end 135.749 124.126) (width 0.3) (layer "F.Cu") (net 3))
 (segment (start 136 128.5) (end 135.749 128.249) (width 0.3) (layer "F.Cu") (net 3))
 (segment (start 135.75 115.25) (end 135.499 114.999) (width 0.3) (layer "F.Cu") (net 3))
 (segment (start 128.5 128.5) (end 128.249 128.249) (width 0.3) (layer "F.Cu") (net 3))
 (segment (start 128.249 110.876) (end 129.125 110) (width 0.3) (layer "F.Cu") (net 3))
 (segment (start 128.249 124.126) (end 129.125 123.25) (width 0.3) (layer "F.Cu") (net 3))
 (segment (start 143.25 128.5) (end 142.999 128.249) (width 0.3) (layer "F.Cu") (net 3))
 (segment (start 128.5 115.25) (end 128.249 114.999) (width 0.3) (layer "F.Cu") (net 3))
 (segment (start 142.999 128.249) (end 142.999 124.126) (width 0.3) (layer "F.Cu") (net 3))
 (segment (start 142.749 114.999) (end 142.749 110.876) (width 0.3) (layer "F.Cu") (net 3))
 (segment (start 135.749 124.126) (end 136.625 123.25) (width 0.3) (layer "F.Cu") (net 3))
 (segment (start 128.249 114.999) (end 128.249 110.876) (width 0.3) (layer "F.Cu") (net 3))
 (segment (start 128.249 128.249) (end 128.249 124.126) (width 0.3) (layer "F.Cu") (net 3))
 (segment (start 143 115.25) (end 142.749 114.999) (width 0.3) (layer "F.Cu") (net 3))
 (segment (start 135.499 114.999) (end 135.499 110.876) (width 0.3) (layer "F.Cu") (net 3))
 (segment (start 142.999 124.126) (end 143.875 123.25) (width 0.3) (layer "F.Cu") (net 3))
 (segment (start 137 127.125) (end 136.625 126.75) (width 0.3) (layer "F.Cu") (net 1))
 (segment (start 129.5 128.5) (end 129.5 127.125) (width 0.3) (layer "F.Cu") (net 1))
 (segment (start 136.75 113.875) (end 136.375 113.5) (width 0.3) (layer "F.Cu") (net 1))
 (segment (start 144 115.25) (end 144 113.875) (width 0.3) (layer "F.Cu") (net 1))
 (segment (start 144 113.875) (end 143.625 113.5) (width 0.3) (layer "F.Cu") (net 1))
 (segment (start 129.5 113.875) (end 129.125 113.5) (width 0.3) (layer "F.Cu") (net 1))
 (segment (start 144.25 128.5) (end 144.25 127.125) (width 0.3) (layer "F.Cu") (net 1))
 (segment (start 129.5 127.125) (end 129.125 126.75) (width 0.3) (layer "F.Cu") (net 1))
 (segment (start 144.25 127.125) (end 143.875 126.75) (width 0.3) (layer "F.Cu") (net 1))
 (segment (start 136.75 115.25) (end 136.75 113.875) (width 0.3) (layer "F.Cu") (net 1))
 (segment (start 129.5 115.25) (end 129.5 113.875) (width 0.3) (layer "F.Cu") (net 1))
 (segment (start 137 128.5) (end 137 127.125) (width 0.3) (layer "F.Cu") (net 1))
 (segment (start 145.25 128.875) (end 143.875 130.25) (width 0.3) (layer "F.Cu") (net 4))
 (segment (start 130.5 115.25) (end 130.5 115.625) (width 0.3) (layer "F.Cu") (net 4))
 (segment (start 138 128.875) (end 136.625 130.25) (width 0.3) (layer "F.Cu") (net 4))
 (segment (start 130.5 115.625) (end 129.125 117) (width 0.3) (layer "F.Cu") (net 4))
 (segment (start 137.75 115.625) (end 136.375 117) (width 0.3) (layer "F.Cu") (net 4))
 (segment (start 145 115.25) (end 145 115.625) (width 0.3) (layer "F.Cu") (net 4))
 (segment (start 130.5 128.5) (end 130.5 128.875) (width 0.3) (layer "F.Cu") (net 4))
 (segment (start 138 128.5) (end 138 128.875) (width 0.3) (layer "F.Cu") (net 4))
 (segment (start 137.75 115.25) (end 137.75 115.625) (width 0.3) (layer "F.Cu") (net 4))
 (segment (start 145 115.625) (end 143.625 117) (width 0.3) (layer "F.Cu") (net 4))
 (segment (start 145.25 128.5) (end 145.25 128.875) (width 0.3) (layer "F.Cu") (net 4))
 (segment (start 130.5 128.875) (end 129.125 130.25) (width 0.3) (layer "F.Cu") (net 4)))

